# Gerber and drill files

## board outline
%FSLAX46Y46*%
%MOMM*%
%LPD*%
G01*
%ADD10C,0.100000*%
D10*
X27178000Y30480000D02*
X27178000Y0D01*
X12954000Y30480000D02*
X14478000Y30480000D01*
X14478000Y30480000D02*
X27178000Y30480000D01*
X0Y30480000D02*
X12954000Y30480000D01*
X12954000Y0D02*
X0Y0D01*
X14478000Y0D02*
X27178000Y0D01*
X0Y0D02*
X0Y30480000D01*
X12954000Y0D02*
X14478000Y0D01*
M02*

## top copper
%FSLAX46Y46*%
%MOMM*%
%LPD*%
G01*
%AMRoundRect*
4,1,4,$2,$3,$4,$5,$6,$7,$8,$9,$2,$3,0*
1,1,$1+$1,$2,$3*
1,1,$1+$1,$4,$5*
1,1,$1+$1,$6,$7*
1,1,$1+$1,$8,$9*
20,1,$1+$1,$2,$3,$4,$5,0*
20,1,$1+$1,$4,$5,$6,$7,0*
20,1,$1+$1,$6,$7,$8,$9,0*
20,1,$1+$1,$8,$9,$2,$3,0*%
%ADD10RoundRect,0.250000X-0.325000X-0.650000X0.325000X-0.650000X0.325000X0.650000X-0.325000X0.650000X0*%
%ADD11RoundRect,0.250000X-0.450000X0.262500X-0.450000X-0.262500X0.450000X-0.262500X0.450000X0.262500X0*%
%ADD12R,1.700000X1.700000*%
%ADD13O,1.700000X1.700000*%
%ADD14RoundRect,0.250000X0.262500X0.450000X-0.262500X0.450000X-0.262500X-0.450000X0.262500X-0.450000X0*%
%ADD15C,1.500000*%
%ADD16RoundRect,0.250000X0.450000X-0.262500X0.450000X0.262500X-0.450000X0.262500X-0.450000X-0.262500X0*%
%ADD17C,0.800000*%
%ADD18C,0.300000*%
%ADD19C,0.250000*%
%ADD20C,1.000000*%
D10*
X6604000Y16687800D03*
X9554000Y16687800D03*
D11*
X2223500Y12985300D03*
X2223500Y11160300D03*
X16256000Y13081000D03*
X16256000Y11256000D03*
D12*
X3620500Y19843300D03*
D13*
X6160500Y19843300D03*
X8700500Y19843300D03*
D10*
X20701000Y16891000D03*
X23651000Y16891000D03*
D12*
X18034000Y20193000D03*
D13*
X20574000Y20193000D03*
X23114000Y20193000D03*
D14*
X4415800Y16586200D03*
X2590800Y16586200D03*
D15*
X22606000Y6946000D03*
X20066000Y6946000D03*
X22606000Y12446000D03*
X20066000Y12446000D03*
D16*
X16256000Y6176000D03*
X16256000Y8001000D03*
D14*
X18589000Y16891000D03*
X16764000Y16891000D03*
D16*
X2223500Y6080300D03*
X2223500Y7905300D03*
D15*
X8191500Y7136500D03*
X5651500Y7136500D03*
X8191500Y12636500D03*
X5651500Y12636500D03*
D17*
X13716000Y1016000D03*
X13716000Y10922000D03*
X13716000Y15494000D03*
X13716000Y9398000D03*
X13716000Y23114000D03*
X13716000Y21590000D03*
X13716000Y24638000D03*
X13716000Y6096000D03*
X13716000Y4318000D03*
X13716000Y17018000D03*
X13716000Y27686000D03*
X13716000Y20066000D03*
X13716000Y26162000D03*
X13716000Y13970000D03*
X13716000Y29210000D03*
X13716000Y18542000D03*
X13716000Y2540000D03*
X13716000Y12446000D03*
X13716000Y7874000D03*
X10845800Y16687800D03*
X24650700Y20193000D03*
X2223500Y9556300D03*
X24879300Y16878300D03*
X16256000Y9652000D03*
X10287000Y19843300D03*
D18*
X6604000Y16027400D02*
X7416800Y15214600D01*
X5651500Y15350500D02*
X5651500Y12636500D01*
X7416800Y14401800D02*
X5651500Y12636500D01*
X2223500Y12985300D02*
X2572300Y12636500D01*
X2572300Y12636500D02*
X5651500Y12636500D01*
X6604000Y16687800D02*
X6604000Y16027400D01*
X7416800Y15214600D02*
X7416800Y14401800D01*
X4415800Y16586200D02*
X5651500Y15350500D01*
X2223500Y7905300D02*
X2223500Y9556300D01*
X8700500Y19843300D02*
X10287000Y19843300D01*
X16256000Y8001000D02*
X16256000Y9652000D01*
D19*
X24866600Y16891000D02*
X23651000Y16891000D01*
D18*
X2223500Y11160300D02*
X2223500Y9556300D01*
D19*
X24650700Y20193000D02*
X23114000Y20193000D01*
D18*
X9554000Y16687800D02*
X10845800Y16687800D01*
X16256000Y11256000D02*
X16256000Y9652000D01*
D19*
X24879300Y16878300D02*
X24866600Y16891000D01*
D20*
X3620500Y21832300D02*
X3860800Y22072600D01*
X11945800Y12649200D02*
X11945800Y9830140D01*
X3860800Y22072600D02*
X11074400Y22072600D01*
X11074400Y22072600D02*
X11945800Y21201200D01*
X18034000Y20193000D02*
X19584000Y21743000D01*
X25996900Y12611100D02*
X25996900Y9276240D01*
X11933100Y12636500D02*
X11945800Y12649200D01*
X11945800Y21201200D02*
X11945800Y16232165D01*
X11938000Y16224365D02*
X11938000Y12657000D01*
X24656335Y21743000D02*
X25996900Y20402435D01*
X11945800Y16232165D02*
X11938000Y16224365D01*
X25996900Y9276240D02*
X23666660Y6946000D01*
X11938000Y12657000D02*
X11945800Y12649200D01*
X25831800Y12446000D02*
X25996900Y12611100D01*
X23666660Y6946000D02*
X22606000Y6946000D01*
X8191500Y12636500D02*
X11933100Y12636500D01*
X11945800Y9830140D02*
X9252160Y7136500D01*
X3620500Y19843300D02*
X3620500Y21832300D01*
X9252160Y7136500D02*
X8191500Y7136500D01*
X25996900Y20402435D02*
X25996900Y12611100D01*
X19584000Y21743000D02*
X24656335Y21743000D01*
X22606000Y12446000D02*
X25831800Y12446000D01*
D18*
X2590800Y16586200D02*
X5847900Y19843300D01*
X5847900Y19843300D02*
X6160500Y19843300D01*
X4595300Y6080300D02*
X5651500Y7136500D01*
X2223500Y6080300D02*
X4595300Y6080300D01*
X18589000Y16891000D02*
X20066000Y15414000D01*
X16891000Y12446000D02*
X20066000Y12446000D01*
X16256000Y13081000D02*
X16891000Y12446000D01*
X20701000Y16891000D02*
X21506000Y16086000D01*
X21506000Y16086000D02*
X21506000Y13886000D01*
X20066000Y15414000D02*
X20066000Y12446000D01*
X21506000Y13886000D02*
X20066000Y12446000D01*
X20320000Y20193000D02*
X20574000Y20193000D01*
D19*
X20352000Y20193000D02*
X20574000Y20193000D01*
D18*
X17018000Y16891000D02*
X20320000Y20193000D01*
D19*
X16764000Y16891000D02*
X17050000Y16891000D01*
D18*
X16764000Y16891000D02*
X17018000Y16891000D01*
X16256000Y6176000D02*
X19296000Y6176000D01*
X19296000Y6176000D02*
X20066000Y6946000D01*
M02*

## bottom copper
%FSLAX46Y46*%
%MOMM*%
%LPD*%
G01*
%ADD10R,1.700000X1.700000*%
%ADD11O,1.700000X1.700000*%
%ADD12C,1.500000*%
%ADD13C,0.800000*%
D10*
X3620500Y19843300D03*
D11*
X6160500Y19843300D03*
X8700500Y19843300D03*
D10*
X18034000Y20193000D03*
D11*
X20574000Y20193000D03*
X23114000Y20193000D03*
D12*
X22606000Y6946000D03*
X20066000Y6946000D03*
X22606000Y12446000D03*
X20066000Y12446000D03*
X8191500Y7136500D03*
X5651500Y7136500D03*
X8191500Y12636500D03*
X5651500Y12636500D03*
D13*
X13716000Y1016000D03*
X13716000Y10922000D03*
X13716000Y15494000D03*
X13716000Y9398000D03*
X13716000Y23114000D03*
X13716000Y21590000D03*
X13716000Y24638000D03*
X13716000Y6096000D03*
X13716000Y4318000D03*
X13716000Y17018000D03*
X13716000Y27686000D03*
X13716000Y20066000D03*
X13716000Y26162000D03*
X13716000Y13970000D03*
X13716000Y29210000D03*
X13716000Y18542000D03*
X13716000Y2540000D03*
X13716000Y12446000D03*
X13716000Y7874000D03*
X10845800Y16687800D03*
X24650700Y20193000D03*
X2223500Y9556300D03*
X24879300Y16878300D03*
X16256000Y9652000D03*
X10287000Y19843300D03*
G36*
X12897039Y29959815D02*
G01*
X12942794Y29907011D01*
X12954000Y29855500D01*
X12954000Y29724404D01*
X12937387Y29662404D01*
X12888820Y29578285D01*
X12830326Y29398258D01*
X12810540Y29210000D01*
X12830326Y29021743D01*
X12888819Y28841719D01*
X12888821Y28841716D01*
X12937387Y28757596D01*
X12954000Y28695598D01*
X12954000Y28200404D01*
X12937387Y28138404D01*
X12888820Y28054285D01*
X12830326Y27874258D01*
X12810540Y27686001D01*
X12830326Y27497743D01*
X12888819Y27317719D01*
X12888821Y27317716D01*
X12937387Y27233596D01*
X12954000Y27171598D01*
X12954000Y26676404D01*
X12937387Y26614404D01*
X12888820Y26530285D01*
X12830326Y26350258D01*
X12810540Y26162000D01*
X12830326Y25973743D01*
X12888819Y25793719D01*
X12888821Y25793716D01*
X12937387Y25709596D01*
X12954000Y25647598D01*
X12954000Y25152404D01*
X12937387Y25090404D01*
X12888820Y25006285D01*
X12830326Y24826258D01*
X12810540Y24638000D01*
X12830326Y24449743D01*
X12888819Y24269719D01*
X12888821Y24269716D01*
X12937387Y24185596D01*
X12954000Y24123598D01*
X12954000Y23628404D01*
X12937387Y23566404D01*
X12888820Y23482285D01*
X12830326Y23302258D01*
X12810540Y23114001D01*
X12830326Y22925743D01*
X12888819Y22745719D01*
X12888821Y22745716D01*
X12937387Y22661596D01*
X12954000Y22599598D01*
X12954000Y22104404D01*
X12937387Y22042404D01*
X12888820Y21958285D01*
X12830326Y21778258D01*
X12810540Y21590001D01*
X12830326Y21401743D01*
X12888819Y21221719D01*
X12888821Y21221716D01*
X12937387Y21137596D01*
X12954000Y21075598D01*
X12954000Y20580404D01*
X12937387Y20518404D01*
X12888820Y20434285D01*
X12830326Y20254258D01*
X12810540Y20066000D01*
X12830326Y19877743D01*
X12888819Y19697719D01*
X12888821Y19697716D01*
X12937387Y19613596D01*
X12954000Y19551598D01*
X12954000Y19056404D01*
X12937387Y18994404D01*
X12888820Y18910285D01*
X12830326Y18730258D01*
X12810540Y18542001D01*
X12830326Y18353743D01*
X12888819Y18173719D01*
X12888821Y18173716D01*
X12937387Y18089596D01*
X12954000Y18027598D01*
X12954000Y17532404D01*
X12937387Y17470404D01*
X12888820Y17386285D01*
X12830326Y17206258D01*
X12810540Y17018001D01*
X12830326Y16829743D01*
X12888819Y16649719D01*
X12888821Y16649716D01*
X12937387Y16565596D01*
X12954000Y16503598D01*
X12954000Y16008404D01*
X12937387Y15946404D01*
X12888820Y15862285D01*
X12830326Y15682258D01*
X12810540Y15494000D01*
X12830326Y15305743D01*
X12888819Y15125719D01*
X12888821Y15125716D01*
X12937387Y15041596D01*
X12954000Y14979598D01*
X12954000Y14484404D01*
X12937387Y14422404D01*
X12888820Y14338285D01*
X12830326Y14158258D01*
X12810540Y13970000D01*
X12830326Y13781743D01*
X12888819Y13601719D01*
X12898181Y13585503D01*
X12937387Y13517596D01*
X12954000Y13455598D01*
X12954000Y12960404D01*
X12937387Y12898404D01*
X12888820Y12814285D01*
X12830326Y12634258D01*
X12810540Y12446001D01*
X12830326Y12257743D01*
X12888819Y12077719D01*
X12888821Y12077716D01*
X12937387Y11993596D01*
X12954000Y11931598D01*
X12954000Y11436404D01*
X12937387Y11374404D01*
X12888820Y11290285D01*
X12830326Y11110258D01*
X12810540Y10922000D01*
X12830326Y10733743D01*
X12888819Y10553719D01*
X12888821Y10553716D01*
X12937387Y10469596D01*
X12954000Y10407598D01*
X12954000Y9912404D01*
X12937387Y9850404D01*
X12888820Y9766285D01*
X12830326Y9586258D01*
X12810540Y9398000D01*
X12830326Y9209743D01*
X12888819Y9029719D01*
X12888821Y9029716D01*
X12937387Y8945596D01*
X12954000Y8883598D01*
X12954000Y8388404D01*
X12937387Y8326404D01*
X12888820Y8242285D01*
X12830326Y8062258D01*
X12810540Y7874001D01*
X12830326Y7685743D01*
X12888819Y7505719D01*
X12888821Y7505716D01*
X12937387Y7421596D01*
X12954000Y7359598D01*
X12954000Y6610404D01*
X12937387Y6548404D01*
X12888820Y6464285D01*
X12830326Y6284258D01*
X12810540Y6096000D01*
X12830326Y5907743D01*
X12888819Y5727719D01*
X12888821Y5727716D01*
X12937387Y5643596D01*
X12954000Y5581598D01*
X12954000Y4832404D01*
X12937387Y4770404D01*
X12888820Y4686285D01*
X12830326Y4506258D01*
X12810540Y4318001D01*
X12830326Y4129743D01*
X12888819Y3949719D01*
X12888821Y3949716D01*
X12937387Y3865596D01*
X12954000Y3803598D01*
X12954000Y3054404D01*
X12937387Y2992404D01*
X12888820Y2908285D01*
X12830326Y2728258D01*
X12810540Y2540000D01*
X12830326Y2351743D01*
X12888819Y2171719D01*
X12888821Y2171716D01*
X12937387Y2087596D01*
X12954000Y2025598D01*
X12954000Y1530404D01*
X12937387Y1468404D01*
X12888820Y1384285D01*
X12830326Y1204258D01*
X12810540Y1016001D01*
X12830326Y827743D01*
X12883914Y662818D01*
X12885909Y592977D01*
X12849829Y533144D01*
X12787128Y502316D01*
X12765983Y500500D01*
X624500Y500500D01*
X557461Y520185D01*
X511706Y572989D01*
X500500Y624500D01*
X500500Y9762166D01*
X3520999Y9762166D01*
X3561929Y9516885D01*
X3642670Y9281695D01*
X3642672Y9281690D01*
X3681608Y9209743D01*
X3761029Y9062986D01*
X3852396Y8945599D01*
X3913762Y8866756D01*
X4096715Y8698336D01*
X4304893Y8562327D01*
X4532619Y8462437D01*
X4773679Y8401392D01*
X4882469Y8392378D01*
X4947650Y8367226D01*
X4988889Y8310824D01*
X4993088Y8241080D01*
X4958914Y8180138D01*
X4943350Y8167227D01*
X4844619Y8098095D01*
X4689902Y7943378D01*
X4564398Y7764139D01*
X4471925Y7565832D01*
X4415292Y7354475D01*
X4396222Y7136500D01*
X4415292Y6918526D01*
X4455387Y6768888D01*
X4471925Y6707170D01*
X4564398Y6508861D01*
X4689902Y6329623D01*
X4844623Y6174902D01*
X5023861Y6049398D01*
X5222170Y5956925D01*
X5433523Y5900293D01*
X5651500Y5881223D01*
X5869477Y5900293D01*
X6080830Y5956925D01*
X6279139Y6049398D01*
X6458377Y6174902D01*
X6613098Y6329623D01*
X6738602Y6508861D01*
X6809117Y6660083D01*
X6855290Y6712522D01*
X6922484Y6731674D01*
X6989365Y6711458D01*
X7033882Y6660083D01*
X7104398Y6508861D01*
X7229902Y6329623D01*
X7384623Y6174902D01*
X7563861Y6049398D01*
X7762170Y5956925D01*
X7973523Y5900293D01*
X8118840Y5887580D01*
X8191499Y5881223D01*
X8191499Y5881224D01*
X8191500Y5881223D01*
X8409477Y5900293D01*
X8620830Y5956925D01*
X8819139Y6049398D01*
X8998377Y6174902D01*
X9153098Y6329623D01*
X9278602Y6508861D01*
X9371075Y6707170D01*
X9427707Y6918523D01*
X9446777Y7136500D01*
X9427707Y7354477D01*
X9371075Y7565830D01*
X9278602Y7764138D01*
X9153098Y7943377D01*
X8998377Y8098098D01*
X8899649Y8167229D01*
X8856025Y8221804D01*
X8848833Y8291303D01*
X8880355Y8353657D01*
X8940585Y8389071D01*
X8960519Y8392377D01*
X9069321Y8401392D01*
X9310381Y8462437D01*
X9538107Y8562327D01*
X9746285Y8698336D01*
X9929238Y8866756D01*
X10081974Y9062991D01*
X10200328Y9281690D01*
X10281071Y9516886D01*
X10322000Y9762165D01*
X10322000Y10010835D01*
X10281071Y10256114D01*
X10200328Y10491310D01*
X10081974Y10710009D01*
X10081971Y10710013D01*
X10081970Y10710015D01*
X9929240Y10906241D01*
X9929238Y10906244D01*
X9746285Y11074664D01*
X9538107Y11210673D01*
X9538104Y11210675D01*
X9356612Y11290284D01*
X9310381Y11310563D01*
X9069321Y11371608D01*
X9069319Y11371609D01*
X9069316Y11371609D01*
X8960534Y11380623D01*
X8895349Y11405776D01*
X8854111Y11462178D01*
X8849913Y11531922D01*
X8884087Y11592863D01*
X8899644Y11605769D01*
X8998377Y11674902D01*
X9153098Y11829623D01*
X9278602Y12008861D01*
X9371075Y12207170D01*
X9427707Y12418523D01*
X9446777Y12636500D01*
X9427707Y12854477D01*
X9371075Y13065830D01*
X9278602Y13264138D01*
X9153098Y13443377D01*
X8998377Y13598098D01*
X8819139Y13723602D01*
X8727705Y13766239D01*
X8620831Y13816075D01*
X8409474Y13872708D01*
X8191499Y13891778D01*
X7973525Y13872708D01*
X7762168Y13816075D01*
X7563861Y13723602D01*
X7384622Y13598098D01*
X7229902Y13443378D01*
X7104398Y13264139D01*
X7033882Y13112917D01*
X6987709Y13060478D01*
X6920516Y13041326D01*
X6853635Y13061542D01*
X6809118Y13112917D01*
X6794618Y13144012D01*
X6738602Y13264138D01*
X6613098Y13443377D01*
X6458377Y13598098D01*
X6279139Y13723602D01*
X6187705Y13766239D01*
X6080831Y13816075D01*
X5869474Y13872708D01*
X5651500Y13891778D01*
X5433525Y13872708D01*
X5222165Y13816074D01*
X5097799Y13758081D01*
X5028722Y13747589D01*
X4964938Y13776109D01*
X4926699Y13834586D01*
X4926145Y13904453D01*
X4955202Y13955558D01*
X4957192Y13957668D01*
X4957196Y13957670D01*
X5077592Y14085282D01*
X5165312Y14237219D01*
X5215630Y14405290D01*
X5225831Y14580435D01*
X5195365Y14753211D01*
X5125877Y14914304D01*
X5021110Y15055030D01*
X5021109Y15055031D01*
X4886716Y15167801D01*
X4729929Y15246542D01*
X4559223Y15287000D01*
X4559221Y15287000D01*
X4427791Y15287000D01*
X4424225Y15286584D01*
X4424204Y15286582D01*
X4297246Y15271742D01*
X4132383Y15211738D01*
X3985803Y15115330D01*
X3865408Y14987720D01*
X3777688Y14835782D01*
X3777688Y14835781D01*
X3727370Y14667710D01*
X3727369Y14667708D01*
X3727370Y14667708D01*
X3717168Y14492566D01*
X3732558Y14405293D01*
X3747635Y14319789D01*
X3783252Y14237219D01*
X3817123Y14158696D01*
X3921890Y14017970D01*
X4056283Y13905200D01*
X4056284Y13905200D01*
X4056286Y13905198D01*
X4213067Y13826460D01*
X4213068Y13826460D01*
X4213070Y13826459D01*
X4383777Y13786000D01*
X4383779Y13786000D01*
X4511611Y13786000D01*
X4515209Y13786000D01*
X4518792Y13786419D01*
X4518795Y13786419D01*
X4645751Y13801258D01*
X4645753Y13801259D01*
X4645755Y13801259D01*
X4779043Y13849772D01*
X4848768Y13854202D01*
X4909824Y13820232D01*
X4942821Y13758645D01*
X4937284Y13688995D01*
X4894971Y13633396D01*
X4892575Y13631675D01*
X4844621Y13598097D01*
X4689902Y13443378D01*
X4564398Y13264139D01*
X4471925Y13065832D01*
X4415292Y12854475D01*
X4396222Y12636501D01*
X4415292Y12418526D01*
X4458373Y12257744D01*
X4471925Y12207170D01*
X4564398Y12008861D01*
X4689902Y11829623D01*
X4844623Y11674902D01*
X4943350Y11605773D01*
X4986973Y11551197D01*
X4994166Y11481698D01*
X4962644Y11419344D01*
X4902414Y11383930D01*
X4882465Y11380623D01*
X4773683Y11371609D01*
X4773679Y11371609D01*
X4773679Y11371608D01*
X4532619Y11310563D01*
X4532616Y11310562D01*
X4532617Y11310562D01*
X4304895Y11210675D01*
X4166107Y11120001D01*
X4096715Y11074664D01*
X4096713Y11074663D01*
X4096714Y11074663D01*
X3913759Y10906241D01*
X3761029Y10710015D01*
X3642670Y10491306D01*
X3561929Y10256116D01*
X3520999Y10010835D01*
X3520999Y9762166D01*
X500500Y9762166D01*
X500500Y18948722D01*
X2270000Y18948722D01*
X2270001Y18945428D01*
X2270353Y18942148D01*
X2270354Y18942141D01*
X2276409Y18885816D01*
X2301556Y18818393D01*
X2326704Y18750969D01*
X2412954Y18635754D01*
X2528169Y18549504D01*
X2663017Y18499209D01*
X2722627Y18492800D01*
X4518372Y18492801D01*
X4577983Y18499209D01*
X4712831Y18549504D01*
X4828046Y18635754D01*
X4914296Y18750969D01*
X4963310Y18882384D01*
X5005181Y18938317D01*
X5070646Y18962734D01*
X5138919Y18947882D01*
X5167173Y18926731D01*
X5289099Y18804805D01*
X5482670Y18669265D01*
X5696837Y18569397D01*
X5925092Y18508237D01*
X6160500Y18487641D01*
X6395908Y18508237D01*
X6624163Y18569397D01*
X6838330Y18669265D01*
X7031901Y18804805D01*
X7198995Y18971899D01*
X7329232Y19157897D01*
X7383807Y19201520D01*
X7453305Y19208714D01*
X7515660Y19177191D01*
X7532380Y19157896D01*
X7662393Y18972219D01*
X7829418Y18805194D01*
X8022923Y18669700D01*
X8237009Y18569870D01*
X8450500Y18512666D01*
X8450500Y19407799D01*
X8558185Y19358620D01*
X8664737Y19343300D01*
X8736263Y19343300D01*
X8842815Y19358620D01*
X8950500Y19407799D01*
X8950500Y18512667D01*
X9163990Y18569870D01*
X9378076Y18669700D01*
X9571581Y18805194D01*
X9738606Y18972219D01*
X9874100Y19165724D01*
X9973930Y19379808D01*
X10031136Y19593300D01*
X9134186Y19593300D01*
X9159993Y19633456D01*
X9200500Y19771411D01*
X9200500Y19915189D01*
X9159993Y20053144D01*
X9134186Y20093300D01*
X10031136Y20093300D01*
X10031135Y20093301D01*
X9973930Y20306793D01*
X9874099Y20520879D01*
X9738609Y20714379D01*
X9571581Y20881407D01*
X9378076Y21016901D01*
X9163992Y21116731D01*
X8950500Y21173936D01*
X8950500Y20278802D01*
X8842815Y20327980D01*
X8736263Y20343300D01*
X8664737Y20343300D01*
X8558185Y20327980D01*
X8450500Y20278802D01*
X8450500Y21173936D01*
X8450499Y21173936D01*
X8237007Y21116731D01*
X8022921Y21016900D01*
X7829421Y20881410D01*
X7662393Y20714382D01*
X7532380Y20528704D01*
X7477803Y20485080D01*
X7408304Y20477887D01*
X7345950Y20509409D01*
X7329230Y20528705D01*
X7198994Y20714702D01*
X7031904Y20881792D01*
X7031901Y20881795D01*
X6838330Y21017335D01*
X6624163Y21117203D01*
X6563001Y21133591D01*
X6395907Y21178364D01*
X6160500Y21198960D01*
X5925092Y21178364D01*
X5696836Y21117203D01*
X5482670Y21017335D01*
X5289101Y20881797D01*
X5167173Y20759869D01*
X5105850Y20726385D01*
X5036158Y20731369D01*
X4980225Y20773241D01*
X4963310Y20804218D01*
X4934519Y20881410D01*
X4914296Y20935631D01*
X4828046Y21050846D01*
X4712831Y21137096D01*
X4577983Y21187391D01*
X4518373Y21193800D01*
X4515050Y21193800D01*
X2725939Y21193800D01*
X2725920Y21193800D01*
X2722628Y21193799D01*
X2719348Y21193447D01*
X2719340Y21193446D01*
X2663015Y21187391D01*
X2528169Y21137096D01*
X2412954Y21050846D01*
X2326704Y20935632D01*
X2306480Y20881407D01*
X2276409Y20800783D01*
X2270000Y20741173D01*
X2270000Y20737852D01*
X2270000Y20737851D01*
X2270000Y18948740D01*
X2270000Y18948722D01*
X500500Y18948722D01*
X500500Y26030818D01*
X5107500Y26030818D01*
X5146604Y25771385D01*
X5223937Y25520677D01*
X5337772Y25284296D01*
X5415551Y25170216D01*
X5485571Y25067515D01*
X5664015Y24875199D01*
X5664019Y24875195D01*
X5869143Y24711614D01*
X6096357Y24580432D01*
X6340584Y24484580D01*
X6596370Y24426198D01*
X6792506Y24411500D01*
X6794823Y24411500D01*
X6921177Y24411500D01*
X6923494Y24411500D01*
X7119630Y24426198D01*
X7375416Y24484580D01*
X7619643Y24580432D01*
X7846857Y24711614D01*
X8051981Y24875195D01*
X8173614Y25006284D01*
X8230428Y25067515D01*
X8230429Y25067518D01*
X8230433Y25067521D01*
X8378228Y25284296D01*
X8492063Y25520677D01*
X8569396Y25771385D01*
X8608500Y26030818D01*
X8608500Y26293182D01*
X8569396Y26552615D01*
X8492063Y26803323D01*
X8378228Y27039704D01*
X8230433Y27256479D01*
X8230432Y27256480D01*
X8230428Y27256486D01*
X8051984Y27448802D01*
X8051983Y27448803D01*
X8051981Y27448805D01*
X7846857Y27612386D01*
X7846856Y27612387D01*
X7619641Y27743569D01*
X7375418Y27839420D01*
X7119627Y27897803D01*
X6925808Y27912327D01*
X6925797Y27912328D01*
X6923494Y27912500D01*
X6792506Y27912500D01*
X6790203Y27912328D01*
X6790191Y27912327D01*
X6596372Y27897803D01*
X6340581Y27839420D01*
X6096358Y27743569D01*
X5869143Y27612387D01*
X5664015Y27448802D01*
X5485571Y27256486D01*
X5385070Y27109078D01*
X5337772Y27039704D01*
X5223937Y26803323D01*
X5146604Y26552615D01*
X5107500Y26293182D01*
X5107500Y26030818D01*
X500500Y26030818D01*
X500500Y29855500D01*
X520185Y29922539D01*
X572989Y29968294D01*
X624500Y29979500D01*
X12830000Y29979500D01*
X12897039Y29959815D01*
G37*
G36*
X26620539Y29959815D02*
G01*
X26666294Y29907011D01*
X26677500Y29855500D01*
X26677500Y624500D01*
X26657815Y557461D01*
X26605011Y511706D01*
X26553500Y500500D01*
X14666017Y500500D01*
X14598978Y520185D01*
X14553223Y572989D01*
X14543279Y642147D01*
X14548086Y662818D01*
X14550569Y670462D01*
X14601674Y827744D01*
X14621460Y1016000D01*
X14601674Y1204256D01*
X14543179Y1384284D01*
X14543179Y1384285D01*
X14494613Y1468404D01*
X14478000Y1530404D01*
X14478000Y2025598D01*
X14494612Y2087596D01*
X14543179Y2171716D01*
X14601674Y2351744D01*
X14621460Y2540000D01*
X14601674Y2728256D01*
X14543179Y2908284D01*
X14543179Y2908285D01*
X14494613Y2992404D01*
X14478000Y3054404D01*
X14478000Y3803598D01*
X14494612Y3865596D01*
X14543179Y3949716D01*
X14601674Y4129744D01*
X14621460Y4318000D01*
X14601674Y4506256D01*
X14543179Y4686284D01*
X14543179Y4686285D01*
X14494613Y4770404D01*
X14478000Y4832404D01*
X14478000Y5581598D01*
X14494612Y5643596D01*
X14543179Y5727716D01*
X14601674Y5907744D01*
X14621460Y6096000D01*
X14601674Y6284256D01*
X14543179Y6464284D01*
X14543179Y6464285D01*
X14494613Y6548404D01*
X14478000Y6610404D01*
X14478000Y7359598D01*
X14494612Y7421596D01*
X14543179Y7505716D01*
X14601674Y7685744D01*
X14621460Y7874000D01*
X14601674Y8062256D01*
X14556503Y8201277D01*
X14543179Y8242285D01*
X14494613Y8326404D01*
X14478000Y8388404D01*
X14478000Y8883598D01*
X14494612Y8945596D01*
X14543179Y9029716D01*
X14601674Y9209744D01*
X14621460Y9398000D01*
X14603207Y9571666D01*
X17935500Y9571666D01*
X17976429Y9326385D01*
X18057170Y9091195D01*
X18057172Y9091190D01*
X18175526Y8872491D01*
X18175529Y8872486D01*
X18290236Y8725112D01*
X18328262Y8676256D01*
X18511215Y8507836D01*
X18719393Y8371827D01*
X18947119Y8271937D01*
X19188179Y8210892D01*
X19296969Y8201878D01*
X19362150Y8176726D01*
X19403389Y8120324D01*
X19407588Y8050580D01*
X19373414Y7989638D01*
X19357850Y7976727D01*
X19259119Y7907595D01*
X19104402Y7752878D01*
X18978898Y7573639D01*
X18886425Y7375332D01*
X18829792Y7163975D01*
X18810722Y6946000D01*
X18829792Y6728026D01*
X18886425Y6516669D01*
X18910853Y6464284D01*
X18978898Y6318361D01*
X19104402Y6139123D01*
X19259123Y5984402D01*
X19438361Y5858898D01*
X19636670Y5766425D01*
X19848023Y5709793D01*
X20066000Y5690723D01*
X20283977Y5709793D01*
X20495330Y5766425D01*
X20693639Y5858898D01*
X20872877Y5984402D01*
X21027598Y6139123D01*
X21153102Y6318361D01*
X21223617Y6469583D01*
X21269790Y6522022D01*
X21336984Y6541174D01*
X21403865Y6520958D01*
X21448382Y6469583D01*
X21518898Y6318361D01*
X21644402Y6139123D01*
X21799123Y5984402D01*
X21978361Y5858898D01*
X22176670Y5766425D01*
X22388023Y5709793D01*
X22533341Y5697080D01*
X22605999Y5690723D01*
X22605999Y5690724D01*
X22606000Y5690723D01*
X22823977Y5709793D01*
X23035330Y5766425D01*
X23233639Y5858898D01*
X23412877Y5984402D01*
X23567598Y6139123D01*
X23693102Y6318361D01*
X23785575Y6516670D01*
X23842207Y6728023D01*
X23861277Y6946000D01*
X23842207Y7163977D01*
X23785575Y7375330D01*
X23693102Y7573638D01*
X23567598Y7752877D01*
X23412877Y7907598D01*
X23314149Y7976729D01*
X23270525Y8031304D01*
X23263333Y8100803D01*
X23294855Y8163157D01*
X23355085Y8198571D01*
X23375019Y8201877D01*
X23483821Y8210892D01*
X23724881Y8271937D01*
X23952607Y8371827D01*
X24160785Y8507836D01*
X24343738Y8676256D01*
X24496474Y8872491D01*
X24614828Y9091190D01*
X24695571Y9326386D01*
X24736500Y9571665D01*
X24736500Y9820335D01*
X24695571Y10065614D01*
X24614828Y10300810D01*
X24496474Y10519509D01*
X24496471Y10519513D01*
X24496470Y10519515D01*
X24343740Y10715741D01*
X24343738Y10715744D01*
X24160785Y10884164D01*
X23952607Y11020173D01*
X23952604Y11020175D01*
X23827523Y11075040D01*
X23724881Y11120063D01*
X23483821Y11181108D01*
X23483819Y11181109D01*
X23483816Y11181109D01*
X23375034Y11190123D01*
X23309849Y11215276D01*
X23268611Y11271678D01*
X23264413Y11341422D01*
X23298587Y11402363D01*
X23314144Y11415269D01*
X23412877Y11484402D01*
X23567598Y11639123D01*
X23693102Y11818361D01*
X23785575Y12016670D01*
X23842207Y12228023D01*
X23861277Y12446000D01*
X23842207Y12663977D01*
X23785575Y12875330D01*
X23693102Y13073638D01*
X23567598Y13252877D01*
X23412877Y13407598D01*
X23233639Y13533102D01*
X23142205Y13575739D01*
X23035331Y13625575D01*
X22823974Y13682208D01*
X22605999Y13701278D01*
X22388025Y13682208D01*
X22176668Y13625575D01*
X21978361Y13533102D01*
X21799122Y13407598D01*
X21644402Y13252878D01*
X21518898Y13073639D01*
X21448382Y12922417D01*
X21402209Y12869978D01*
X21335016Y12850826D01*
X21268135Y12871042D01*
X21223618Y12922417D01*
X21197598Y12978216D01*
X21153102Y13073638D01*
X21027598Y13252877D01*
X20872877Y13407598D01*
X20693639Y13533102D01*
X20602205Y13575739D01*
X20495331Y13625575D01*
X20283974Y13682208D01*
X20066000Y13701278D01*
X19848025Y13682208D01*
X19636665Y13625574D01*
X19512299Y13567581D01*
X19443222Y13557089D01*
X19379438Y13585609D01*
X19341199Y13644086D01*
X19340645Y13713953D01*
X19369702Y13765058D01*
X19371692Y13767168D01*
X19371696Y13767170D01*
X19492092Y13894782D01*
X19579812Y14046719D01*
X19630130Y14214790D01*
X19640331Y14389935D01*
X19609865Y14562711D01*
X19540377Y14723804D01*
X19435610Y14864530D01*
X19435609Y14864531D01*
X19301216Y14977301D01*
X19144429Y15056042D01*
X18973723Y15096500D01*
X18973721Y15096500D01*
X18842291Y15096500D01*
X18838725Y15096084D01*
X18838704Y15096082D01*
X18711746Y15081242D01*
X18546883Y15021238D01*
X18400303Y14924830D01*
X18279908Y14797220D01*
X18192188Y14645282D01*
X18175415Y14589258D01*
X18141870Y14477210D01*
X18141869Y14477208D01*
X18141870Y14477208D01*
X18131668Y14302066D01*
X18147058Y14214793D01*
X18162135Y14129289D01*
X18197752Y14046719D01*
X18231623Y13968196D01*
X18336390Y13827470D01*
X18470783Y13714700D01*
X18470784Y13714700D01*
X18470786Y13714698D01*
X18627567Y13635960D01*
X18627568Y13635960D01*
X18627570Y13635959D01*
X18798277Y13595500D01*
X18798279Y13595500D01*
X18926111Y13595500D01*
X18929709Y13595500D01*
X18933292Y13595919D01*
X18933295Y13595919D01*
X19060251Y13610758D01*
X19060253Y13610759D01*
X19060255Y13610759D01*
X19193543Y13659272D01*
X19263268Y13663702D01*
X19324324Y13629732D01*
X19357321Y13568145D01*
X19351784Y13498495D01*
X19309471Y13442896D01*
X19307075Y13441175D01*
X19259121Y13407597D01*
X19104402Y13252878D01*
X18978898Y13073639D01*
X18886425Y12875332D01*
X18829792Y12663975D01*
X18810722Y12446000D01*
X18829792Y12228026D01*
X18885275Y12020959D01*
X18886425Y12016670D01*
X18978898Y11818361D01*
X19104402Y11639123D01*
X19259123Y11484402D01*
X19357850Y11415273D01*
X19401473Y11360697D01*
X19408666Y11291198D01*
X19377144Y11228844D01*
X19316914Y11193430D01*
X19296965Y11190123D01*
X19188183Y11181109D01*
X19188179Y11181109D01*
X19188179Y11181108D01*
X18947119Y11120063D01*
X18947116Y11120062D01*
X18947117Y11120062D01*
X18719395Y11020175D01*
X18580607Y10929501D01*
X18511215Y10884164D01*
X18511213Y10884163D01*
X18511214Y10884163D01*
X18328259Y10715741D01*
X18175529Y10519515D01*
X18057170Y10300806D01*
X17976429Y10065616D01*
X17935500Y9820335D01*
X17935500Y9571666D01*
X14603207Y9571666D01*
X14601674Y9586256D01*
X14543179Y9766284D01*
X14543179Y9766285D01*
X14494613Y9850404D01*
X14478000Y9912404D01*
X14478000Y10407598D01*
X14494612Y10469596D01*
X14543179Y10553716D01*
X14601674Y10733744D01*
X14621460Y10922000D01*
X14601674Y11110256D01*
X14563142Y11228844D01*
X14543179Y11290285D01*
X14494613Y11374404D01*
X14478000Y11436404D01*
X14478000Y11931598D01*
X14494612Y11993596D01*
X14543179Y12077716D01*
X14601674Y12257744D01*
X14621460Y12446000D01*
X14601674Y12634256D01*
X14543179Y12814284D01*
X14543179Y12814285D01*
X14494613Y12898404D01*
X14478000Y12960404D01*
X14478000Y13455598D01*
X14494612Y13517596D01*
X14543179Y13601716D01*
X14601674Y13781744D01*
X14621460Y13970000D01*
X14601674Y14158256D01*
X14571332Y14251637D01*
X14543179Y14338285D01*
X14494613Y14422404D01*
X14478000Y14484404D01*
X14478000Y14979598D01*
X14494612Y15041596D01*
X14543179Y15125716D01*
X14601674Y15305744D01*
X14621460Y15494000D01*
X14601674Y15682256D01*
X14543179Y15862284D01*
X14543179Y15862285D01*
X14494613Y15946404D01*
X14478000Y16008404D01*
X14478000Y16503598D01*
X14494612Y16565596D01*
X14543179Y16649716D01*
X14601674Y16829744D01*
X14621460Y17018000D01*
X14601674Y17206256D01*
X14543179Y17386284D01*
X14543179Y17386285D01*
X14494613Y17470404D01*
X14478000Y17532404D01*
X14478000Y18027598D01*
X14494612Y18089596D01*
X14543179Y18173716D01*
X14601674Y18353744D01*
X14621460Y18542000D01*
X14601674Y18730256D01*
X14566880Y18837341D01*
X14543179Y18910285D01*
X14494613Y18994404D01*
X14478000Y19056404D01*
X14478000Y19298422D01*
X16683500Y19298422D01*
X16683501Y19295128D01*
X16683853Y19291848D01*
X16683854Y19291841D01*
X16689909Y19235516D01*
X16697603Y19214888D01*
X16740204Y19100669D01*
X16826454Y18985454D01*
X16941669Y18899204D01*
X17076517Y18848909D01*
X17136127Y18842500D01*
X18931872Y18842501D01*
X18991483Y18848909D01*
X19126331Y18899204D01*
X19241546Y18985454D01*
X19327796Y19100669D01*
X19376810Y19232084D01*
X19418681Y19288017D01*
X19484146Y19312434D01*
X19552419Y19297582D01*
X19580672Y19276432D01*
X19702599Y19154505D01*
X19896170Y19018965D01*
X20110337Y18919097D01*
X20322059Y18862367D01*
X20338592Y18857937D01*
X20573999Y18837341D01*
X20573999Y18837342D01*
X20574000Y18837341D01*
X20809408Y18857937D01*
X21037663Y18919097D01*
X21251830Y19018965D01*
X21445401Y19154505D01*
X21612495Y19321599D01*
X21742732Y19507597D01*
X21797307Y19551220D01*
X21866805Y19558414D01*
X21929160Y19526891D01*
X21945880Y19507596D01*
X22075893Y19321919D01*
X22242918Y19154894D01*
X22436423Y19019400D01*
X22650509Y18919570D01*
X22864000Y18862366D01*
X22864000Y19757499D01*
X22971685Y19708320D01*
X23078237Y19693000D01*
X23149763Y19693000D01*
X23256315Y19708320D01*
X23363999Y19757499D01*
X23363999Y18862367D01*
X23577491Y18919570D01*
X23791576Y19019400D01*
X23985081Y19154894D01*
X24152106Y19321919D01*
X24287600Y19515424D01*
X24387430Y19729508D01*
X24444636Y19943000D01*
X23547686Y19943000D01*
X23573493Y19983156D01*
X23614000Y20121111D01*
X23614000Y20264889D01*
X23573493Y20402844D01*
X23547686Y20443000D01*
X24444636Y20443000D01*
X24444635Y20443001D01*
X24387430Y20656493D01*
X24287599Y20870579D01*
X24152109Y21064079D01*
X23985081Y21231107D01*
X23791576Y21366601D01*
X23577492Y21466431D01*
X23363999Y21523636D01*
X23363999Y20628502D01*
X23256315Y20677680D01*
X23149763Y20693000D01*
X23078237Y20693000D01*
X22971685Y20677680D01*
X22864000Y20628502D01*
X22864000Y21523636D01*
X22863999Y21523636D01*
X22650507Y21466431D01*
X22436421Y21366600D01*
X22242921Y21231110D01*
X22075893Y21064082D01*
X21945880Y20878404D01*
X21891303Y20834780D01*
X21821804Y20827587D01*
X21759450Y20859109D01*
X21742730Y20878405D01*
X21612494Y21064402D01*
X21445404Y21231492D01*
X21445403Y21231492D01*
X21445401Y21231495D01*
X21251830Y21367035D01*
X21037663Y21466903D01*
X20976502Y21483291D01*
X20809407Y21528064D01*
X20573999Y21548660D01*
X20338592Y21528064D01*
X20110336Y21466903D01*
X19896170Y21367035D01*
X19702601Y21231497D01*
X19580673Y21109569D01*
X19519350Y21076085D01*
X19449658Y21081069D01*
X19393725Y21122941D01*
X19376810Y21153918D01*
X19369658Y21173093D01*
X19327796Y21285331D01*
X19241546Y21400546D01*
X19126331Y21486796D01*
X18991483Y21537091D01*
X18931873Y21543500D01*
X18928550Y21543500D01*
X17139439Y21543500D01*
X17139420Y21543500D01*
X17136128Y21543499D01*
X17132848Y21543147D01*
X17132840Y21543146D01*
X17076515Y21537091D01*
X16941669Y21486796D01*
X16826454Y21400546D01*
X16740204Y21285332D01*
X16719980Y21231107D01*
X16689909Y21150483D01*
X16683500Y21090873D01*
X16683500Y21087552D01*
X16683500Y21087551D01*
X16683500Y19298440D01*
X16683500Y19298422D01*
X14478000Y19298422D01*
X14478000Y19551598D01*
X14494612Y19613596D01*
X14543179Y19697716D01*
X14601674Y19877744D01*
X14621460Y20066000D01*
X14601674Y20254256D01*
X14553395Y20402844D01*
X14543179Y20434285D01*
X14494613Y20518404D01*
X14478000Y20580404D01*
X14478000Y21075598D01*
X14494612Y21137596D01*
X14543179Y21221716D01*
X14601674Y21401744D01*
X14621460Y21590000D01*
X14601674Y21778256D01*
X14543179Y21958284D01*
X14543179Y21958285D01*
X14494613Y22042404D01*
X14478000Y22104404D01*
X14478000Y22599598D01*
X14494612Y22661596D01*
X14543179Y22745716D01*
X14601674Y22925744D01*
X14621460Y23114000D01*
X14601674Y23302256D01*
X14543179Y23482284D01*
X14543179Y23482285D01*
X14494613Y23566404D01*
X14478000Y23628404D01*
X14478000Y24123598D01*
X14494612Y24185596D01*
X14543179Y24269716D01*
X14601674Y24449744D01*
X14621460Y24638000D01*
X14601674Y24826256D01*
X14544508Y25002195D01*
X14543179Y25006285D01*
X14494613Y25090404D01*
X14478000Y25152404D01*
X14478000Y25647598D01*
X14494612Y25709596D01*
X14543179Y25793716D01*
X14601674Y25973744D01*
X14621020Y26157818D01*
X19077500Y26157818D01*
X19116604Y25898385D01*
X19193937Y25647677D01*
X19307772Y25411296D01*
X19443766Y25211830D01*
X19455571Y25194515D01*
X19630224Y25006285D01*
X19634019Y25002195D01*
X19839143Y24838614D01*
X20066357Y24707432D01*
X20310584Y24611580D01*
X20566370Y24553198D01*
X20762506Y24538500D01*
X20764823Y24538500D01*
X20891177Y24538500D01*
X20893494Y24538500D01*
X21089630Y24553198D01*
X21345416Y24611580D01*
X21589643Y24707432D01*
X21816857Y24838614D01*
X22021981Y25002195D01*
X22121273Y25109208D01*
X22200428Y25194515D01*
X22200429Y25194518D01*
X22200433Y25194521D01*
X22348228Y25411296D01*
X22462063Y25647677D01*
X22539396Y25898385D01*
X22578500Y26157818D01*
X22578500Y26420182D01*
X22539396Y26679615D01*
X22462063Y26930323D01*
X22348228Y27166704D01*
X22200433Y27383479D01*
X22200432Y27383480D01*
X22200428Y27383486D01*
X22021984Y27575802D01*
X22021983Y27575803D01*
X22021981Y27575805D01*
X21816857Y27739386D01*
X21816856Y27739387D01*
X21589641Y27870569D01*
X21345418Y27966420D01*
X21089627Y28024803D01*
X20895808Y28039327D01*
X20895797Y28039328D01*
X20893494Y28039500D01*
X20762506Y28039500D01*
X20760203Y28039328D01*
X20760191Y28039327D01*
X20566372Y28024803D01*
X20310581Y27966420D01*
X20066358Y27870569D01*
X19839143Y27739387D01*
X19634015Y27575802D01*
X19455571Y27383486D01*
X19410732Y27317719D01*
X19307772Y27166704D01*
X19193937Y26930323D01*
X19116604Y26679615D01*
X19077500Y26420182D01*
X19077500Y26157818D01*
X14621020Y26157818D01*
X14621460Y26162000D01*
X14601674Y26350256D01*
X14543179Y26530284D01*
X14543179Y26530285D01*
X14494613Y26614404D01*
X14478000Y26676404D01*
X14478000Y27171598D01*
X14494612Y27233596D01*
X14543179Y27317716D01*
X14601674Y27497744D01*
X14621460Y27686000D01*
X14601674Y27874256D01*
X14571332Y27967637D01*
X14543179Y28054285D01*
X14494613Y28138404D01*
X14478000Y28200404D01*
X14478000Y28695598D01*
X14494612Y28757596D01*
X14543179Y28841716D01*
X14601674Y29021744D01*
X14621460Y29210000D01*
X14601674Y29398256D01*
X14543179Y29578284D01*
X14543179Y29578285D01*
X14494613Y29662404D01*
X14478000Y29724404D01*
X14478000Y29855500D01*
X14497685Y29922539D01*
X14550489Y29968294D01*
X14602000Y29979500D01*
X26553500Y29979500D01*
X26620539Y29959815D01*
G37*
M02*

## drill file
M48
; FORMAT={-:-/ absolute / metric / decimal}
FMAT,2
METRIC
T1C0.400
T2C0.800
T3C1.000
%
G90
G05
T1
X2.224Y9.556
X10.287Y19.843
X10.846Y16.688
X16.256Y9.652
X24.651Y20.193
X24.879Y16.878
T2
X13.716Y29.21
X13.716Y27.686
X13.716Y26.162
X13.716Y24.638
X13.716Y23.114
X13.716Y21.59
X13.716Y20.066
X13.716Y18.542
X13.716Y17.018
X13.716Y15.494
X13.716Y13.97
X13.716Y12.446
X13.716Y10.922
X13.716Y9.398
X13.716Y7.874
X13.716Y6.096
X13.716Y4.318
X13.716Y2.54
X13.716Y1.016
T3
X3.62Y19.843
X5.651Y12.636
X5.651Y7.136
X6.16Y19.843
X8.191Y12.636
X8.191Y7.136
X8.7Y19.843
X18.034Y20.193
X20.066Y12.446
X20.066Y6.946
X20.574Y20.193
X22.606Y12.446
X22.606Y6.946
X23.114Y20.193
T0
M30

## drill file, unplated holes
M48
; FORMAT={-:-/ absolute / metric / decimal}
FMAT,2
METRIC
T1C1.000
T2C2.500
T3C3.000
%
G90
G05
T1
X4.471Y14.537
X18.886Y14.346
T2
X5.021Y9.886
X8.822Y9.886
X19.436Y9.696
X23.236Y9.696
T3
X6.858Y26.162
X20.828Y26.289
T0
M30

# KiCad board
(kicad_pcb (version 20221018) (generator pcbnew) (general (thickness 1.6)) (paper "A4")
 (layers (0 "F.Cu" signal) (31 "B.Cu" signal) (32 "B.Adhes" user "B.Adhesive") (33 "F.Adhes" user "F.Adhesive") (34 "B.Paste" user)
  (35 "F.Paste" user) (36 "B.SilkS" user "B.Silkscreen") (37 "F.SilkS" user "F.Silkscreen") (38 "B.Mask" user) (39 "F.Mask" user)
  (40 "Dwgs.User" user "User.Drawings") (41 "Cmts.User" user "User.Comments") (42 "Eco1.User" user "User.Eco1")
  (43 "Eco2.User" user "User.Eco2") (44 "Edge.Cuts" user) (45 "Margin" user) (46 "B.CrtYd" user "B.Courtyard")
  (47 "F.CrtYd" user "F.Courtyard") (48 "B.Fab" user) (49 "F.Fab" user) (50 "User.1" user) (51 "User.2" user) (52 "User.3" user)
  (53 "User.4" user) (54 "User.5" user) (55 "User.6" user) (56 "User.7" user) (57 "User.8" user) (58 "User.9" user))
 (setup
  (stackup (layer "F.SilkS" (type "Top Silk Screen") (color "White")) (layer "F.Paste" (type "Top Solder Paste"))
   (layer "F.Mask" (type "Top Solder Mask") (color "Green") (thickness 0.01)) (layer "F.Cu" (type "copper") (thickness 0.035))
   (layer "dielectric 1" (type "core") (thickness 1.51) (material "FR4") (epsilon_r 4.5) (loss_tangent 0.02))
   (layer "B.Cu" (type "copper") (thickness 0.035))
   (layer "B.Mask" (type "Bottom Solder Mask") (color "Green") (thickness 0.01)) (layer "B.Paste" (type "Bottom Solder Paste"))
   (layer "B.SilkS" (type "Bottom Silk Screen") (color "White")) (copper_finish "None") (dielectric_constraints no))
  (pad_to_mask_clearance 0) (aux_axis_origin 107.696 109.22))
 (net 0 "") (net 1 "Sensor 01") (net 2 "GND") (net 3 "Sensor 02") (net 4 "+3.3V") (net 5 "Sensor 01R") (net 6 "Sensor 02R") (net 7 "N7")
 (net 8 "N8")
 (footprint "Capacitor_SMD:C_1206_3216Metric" (layer "F.Cu") (at 115.775 92.5322)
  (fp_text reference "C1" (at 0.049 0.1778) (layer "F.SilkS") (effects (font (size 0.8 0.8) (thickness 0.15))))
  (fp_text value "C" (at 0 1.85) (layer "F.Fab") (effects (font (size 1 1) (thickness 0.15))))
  (pad "1" smd roundrect (at -1.475 0) (size 1.15 1.8) (layers "F.Cu" "F.Paste" "F.Mask") (roundrect_rratio 0.2173913043)
   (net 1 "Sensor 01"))
  (pad "2" smd roundrect (at 1.475 0) (size 1.15 1.8) (layers "F.Cu" "F.Paste" "F.Mask") (roundrect_rratio 0.2173913043) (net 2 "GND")))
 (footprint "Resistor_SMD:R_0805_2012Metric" (layer "F.Cu") (at 109.9195 97.1472 -90)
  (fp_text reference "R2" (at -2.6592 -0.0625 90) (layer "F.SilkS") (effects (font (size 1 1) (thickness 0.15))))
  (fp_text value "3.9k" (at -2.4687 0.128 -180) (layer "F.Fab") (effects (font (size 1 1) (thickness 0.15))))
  (pad "1" smd roundrect (at -0.9125 0 270) (size 1.025 1.4) (layers "F.Cu" "F.Paste" "F.Mask") (roundrect_rratio 0.243902439)
   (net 1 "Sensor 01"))
  (pad "2" smd roundrect (at 0.9125 0 270) (size 1.025 1.4) (layers "F.Cu" "F.Paste" "F.Mask") (roundrect_rratio 0.243902439) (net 2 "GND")))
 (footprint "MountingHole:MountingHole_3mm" (layer "F.Cu") (at 114.554 83.058)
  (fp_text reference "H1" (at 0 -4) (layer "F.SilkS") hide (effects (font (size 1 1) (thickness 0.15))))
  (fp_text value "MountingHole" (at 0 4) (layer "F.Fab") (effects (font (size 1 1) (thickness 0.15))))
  (pad "" np_thru_hole circle (at 0 0) (size 3 3) (drill 3) (layers "*.Cu" "*.Mask")))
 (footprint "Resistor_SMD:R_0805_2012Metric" (layer "F.Cu") (at 123.952 97.0515 -90)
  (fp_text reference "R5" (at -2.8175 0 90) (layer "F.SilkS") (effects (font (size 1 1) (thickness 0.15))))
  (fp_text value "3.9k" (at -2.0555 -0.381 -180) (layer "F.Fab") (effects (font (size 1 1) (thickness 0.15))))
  (pad "1" smd roundrect (at -0.9125 0 270) (size 1.025 1.4) (layers "F.Cu" "F.Paste" "F.Mask") (roundrect_rratio 0.243902439)
   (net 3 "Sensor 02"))
  (pad "2" smd roundrect (at 0.9125 0 270) (size 1.025 1.4) (layers "F.Cu" "F.Paste" "F.Mask") (roundrect_rratio 0.243902439) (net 2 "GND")))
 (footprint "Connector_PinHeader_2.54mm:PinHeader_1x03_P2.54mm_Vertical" (layer "F.Cu") (at 111.3165 89.3767 90)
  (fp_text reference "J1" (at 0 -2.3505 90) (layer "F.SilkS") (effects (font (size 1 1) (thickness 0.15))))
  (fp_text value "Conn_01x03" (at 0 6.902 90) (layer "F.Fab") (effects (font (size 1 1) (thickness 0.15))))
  (pad "1" thru_hole rect (at 0 0 90) (size 1.7 1.7) (drill 1) (layers "*.Cu" "*.Mask") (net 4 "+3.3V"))
  (pad "2" thru_hole oval (at 0 2.54 90) (size 1.7 1.7) (drill 1) (layers "*.Cu" "*.Mask") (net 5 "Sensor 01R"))
  (pad "3" thru_hole oval (at 0 5.08 90) (size 1.7 1.7) (drill 1) (layers "*.Cu" "*.Mask") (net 2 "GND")))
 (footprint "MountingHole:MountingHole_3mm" (layer "F.Cu") (at 128.524 82.931)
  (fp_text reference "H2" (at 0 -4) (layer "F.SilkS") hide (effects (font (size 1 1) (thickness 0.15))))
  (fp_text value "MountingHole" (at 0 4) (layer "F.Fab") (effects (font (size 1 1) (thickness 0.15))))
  (pad "" np_thru_hole circle (at 0 0) (size 3 3) (drill 3) (layers "*.Cu" "*.Mask")))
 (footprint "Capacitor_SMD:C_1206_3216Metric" (layer "F.Cu") (at 129.872 92.329)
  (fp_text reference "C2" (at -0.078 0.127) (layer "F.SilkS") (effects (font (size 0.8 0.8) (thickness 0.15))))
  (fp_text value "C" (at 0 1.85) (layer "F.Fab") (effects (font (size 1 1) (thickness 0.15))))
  (pad "1" smd roundrect (at -1.475 0) (size 1.15 1.8) (layers "F.Cu" "F.Paste" "F.Mask") (roundrect_rratio 0.2173913043)
   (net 3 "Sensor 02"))
  (pad "2" smd roundrect (at 1.475 0) (size 1.15 1.8) (layers "F.Cu" "F.Paste" "F.Mask") (roundrect_rratio 0.2173913043) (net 2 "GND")))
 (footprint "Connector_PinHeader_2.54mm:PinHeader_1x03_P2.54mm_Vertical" (layer "F.Cu") (at 125.73 89.027 90)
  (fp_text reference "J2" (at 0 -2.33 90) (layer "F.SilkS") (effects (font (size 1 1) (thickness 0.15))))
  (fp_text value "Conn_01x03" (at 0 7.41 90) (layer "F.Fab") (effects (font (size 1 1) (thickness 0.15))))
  (pad "1" thru_hole rect (at 0 0 90) (size 1.7 1.7) (drill 1) (layers "*.Cu" "*.Mask") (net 4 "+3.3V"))
  (pad "2" thru_hole oval (at 0 2.54 90) (size 1.7 1.7) (drill 1) (layers "*.Cu" "*.Mask") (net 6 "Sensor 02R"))
  (pad "3" thru_hole oval (at 0 5.08 90) (size 1.7 1.7) (drill 1) (layers "*.Cu" "*.Mask") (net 2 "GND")))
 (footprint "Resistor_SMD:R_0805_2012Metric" (layer "F.Cu") (at 111.1993 92.6338 180)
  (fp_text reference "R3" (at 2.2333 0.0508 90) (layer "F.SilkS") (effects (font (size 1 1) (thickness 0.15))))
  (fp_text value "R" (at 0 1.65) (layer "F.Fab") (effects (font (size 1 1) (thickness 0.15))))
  (pad "1" smd roundrect (at -0.9125 0 180) (size 1.025 1.4) (layers "F.Cu" "F.Paste" "F.Mask") (roundrect_rratio 0.243902439)
   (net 1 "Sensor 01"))
  (pad "2" smd roundrect (at 0.9125 0 180) (size 1.025 1.4) (layers "F.Cu" "F.Paste" "F.Mask") (roundrect_rratio 0.243902439)
   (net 5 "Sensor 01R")))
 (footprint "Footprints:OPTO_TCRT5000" (layer "F.Cu") (at 129.032 99.524 -90)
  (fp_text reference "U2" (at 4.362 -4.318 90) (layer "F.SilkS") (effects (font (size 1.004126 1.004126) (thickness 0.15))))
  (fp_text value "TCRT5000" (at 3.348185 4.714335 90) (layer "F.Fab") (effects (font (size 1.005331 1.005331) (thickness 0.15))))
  (pad "" np_thru_hole circle (at -4.65 2.45 270) (size 1 1) (drill 1) (layers "*.Cu" "*.Mask"))
  (pad "" np_thru_hole circle (at 0 -1.9 270) (size 2.5 2.5) (drill 2.5) (layers "*.Cu" "*.Mask"))
  (pad "" np_thru_hole circle (at 0 1.9 270) (size 2.5 2.5) (drill 2.5) (layers "*.Cu" "*.Mask"))
  (pad "A" thru_hole circle (at 2.75 -1.27 270) (size 1.5 1.5) (drill 1) (layers "*.Cu" "*.Mask") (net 4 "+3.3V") (solder_mask_margin 0.102))
  (pad "CATH" thru_hole circle (at 2.75 1.27 270) (size 1.5 1.5) (drill 1) (layers "*.Cu" "*.Mask") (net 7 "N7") (solder_mask_margin 0.102))
  (pad "COLL" thru_hole circle (at -2.75 -1.27 270) (size 1.5 1.5) (drill 1) (layers "*.Cu" "*.Mask") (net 4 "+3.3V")
   (solder_mask_margin 0.102))
  (pad "E" thru_hole circle (at -2.75 1.27 270) (size 1.5 1.5) (drill 1) (layers "*.Cu" "*.Mask") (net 3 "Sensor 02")
   (solder_mask_margin 0.102)))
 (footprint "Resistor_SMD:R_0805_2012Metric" (layer "F.Cu") (at 123.952 102.1315 90)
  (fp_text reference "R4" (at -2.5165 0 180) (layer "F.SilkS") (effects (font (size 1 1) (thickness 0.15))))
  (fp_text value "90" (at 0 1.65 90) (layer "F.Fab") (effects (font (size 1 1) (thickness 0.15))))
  (pad "1" smd roundrect (at -0.9125 0 90) (size 1.025 1.4) (layers "F.Cu" "F.Paste" "F.Mask") (roundrect_rratio 0.243902439) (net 7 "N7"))
  (pad "2" smd roundrect (at 0.9125 0 90) (size 1.025 1.4) (layers "F.Cu" "F.Paste" "F.Mask") (roundrect_rratio 0.243902439) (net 2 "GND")))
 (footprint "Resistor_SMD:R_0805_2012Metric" (layer "F.Cu") (at 125.3725 92.329 180)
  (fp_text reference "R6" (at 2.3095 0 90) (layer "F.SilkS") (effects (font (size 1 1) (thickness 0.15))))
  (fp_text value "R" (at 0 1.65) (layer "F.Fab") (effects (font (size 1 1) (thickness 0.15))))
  (pad "1" smd roundrect (at -0.9125 0 180) (size 1.025 1.4) (layers "F.Cu" "F.Paste" "F.Mask") (roundrect_rratio 0.243902439)
   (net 3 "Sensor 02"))
  (pad "2" smd roundrect (at 0.9125 0 180) (size 1.025 1.4) (layers "F.Cu" "F.Paste" "F.Mask") (roundrect_rratio 0.243902439)
   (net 6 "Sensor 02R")))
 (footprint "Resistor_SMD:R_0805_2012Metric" (layer "F.Cu") (at 109.9195 102.2272 90)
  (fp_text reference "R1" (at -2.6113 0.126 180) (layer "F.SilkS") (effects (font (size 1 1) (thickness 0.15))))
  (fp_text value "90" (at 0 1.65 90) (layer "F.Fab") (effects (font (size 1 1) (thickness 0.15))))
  (pad "1" smd roundrect (at -0.9125 0 90) (size 1.025 1.4) (layers "F.Cu" "F.Paste" "F.Mask") (roundrect_rratio 0.243902439) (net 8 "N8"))
  (pad "2" smd roundrect (at 0.9125 0 90) (size 1.025 1.4) (layers "F.Cu" "F.Paste" "F.Mask") (roundrect_rratio 0.243902439) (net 2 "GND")))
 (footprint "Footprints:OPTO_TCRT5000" (layer "F.Cu") (at 114.6175 99.3335 -90)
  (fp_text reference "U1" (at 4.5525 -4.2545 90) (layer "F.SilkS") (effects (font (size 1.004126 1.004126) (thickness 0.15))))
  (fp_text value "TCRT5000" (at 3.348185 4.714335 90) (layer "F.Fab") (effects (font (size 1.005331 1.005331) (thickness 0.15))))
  (pad "" np_thru_hole circle (at -4.65 2.45 270) (size 1 1) (drill 1) (layers "*.Cu" "*.Mask"))
  (pad "" np_thru_hole circle (at 0 -1.9 270) (size 2.5 2.5) (drill 2.5) (layers "*.Cu" "*.Mask"))
  (pad "" np_thru_hole circle (at 0 1.9 270) (size 2.5 2.5) (drill 2.5) (layers "*.Cu" "*.Mask"))
  (pad "A" thru_hole circle (at 2.75 -1.27 270) (size 1.5 1.5) (drill 1) (layers "*.Cu" "*.Mask") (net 4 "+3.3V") (solder_mask_margin 0.102))
  (pad "CATH" thru_hole circle (at 2.75 1.27 270) (size 1.5 1.5) (drill 1) (layers "*.Cu" "*.Mask") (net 8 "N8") (solder_mask_margin 0.102))
  (pad "COLL" thru_hole circle (at -2.75 -1.27 270) (size 1.5 1.5) (drill 1) (layers "*.Cu" "*.Mask") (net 4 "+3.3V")
   (solder_mask_margin 0.102))
  (pad "E" thru_hole circle (at -2.75 1.27 270) (size 1.5 1.5) (drill 1) (layers "*.Cu" "*.Mask") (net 1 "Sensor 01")
   (solder_mask_margin 0.102)))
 (gr_line (start 134.874 78.74) (end 134.874 109.22) (stroke (width 0.1) (type default)) (layer "Edge.Cuts"))
 (gr_line (start 120.65 78.74) (end 122.174 78.74) (stroke (width 0.1) (type default)) (layer "Edge.Cuts"))
 (gr_line (start 122.174 78.74) (end 134.874 78.74) (stroke (width 0.1) (type default)) (layer "Edge.Cuts"))
 (gr_line (start 107.696 78.74) (end 120.65 78.74) (stroke (width 0.1) (type default)) (layer "Edge.Cuts"))
 (gr_line (start 120.65 109.22) (end 107.696 109.22) (stroke (width 0.1) (type default)) (layer "Edge.Cuts"))
 (gr_line (start 122.174 109.22) (end 134.874 109.22) (stroke (width 0.1) (type default)) (layer "Edge.Cuts"))
 (gr_line (start 107.696 109.22) (end 107.696 78.74) (stroke (width 0.1) (type default)) (layer "Edge.Cuts"))
 (gr_line (start 120.65 109.22) (end 122.174 109.22) (stroke (width 0.1) (type default)) (layer "Edge.Cuts"))
 (via (at 121.412 108.204) (size 0.8) (drill 0.8) (layers "F.Cu" "B.Cu") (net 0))
 (via (at 121.412 98.298) (size 0.8) (drill 0.8) (layers "F.Cu" "B.Cu") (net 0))
 (via (at 121.412 93.726) (size 0.8) (drill 0.8) (layers "F.Cu" "B.Cu") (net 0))
 (via (at 121.412 99.822) (size 0.8) (drill 0.8) (layers "F.Cu" "B.Cu") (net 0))
 (via (at 121.412 86.106) (size 0.8) (drill 0.8) (layers "F.Cu" "B.Cu") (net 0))
 (via (at 121.412 87.63) (size 0.8) (drill 0.8) (layers "F.Cu" "B.Cu") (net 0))
 (via (at 121.412 84.582) (size 0.8) (drill 0.8) (layers "F.Cu" "B.Cu") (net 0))
 (via (at 121.412 103.124) (size 0.8) (drill 0.8) (layers "F.Cu" "B.Cu") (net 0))
 (via (at 121.412 104.902) (size 0.8) (drill 0.8) (layers "F.Cu" "B.Cu") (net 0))
 (via (at 121.412 92.202) (size 0.8) (drill 0.8) (layers "F.Cu" "B.Cu") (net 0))
 (via (at 121.412 81.534) (size 0.8) (drill 0.8) (layers "F.Cu" "B.Cu") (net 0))
 (via (at 121.412 89.154) (size 0.8) (drill 0.8) (layers "F.Cu" "B.Cu") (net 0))
 (via (at 121.412 83.058) (size 0.8) (drill 0.8) (layers "F.Cu" "B.Cu") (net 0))
 (via (at 121.412 95.25) (size 0.8) (drill 0.8) (layers "F.Cu" "B.Cu") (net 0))
 (via (at 121.412 80.01) (size 0.8) (drill 0.8) (layers "F.Cu" "B.Cu") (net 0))
 (via (at 121.412 90.678) (size 0.8) (drill 0.8) (layers "F.Cu" "B.Cu") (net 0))
 (via (at 121.412 106.68) (size 0.8) (drill 0.8) (layers "F.Cu" "B.Cu") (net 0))
 (via (at 121.412 96.774) (size 0.8) (drill 0.8) (layers "F.Cu" "B.Cu") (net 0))
 (via (at 121.412 101.346) (size 0.8) (drill 0.8) (layers "F.Cu" "B.Cu") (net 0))
 (segment (start 114.3 93.1926) (end 115.1128 94.0054) (width 0.3) (layer "F.Cu") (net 1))
 (segment (start 113.3475 93.8695) (end 113.3475 96.5835) (width 0.3) (layer "F.Cu") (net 1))
 (segment (start 115.1128 94.8182) (end 113.3475 96.5835) (width 0.3) (layer "F.Cu") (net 1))
 (segment (start 109.9195 96.2347) (end 110.2683 96.5835) (width 0.3) (layer "F.Cu") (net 1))
 (segment (start 110.2683 96.5835) (end 113.3475 96.5835) (width 0.3) (layer "F.Cu") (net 1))
 (segment (start 114.3 92.5322) (end 114.3 93.1926) (width 0.3) (layer "F.Cu") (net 1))
 (segment (start 115.1128 94.0054) (end 115.1128 94.8182) (width 0.3) (layer "F.Cu") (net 1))
 (segment (start 112.1118 92.6338) (end 113.3475 93.8695) (width 0.3) (layer "F.Cu") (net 1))
 (segment (start 109.9195 101.3147) (end 109.9195 99.6637) (width 0.3) (layer "F.Cu") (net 2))
 (segment (start 116.3965 89.3767) (end 117.983 89.3767) (width 0.3) (layer "F.Cu") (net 2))
 (segment (start 123.952 101.219) (end 123.952 99.568) (width 0.3) (layer "F.Cu") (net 2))
 (segment (start 132.5626 92.329) (end 131.347 92.329) (width 0.25) (layer "F.Cu") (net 2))
 (segment (start 109.9195 98.0597) (end 109.9195 99.6637) (width 0.3) (layer "F.Cu") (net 2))
 (segment (start 132.3467 89.027) (end 130.81 89.027) (width 0.25) (layer "F.Cu") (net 2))
 (segment (start 117.25 92.5322) (end 118.5418 92.5322) (width 0.3) (layer "F.Cu") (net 2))
 (segment (start 123.952 97.964) (end 123.952 99.568) (width 0.3) (layer "F.Cu") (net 2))
 (segment (start 132.5753 92.3417) (end 132.5626 92.329) (width 0.25) (layer "F.Cu") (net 2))
 (via (at 118.5418 92.5322) (size 0.8) (drill 0.4) (layers "F.Cu" "B.Cu") (free) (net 2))
 (via (at 132.3467 89.027) (size 0.8) (drill 0.4) (layers "F.Cu" "B.Cu") (free) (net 2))
 (via (at 109.9195 99.6637) (size 0.8) (drill 0.4) (layers "F.Cu" "B.Cu") (free) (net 2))
 (via (at 132.5753 92.3417) (size 0.8) (drill 0.4) (layers "F.Cu" "B.Cu") (free) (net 2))
 (via (at 123.952 99.568) (size 0.8) (drill 0.4) (layers "F.Cu" "B.Cu") (free) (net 2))
 (via (at 117.983 89.3767) (size 0.8) (drill 0.4) (layers "F.Cu" "B.Cu") (free) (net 2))
 (segment (start 111.3165 87.3877) (end 111.5568 87.1474) (width 1) (layer "F.Cu") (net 4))
 (segment (start 119.6418 96.5708) (end 119.6418 99.38986) (width 1) (layer "F.Cu") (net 4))
 (segment (start 111.5568 87.1474) (end 118.7704 87.1474) (width 1) (layer "F.Cu") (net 4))
 (segment (start 118.7704 87.1474) (end 119.6418 88.0188) (width 1) (layer "F.Cu") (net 4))
 (segment (start 125.73 89.027) (end 127.28 87.477) (width 1) (layer "F.Cu") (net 4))
 (segment (start 133.6929 96.6089) (end 133.6929 99.94376) (width 1) (layer "F.Cu") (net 4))
 (segment (start 119.6291 96.5835) (end 119.6418 96.5708) (width 1) (layer "F.Cu") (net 4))
 (segment (start 119.6418 88.0188) (end 119.6418 92.987835) (width 1) (layer "F.Cu") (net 4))
 (segment (start 119.634 92.995635) (end 119.634 96.563) (width 1) (layer "F.Cu") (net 4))
 (segment (start 132.352335 87.477) (end 133.6929 88.817565) (width 1) (layer "F.Cu") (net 4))
 (segment (start 119.6418 92.987835) (end 119.634 92.995635) (width 1) (layer "F.Cu") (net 4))
 (segment (start 133.6929 99.94376) (end 131.36266 102.274) (width 1) (layer "F.Cu") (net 4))
 (segment (start 119.634 96.563) (end 119.6418 96.5708) (width 1) (layer "F.Cu") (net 4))
 (segment (start 133.5278 96.774) (end 133.6929 96.6089) (width 1) (layer "F.Cu") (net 4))
 (segment (start 131.36266 102.274) (end 130.302 102.274) (width 1) (layer "F.Cu") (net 4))
 (segment (start 115.8875 96.5835) (end 119.6291 96.5835) (width 1) (layer "F.Cu") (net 4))
 (segment (start 119.6418 99.38986) (end 116.94816 102.0835) (width 1) (layer "F.Cu") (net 4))
 (segment (start 111.3165 89.3767) (end 111.3165 87.3877) (width 1) (layer "F.Cu") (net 4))
 (segment (start 116.94816 102.0835) (end 115.8875 102.0835) (width 1) (layer "F.Cu") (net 4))
 (segment (start 133.6929 88.817565) (end 133.6929 96.6089) (width 1) (layer "F.Cu") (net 4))
 (segment (start 127.28 87.477) (end 132.352335 87.477) (width 1) (layer "F.Cu") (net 4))
 (segment (start 130.302 96.774) (end 133.5278 96.774) (width 1) (layer "F.Cu") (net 4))
 (segment (start 110.2868 92.6338) (end 113.5439 89.3767) (width 0.3) (layer "F.Cu") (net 5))
 (segment (start 113.5439 89.3767) (end 113.8565 89.3767) (width 0.3) (layer "F.Cu") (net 5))
 (segment (start 112.2913 103.1397) (end 113.3475 102.0835) (width 0.3) (layer "F.Cu") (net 8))
 (segment (start 109.9195 103.1397) (end 112.2913 103.1397) (width 0.3) (layer "F.Cu") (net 8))
 (segment (start 126.285 92.329) (end 127.762 93.806) (width 0.3) (layer "F.Cu") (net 3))
 (segment (start 124.587 96.774) (end 127.762 96.774) (width 0.3) (layer "F.Cu") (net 3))
 (segment (start 123.952 96.139) (end 124.587 96.774) (width 0.3) (layer "F.Cu") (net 3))
 (segment (start 128.397 92.329) (end 129.202 93.134) (width 0.3) (layer "F.Cu") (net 3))
 (segment (start 129.202 93.134) (end 129.202 95.334) (width 0.3) (layer "F.Cu") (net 3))
 (segment (start 127.762 93.806) (end 127.762 96.774) (width 0.3) (layer "F.Cu") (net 3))
 (segment (start 129.202 95.334) (end 127.762 96.774) (width 0.3) (layer "F.Cu") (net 3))
 (segment (start 128.016 89.027) (end 128.27 89.027) (width 0.3) (layer "F.Cu") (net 6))
 (segment (start 128.048 89.027) (end 128.27 89.027) (width 0.25) (layer "F.Cu") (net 6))
 (segment (start 124.714 92.329) (end 128.016 89.027) (width 0.3) (layer "F.Cu") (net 6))
 (segment (start 124.46 92.329) (end 124.746 92.329) (width 0.25) (layer "F.Cu") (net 6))
 (segment (start 124.46 92.329) (end 124.714 92.329) (width 0.3) (layer "F.Cu") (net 6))
 (segment (start 123.952 103.044) (end 126.992 103.044) (width 0.3) (layer "F.Cu") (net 7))
 (segment (start 126.992 103.044) (end 127.762 102.274) (width 0.3) (layer "F.Cu") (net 7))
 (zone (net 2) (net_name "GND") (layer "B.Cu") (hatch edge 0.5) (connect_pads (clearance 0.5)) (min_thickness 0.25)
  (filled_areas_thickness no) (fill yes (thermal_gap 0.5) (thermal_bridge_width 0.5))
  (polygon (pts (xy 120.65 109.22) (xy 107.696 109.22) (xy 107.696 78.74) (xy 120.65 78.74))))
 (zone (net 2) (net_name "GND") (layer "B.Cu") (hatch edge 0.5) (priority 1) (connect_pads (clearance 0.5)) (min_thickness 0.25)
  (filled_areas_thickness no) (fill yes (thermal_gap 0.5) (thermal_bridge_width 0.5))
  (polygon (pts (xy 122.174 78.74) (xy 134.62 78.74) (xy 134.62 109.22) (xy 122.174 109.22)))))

